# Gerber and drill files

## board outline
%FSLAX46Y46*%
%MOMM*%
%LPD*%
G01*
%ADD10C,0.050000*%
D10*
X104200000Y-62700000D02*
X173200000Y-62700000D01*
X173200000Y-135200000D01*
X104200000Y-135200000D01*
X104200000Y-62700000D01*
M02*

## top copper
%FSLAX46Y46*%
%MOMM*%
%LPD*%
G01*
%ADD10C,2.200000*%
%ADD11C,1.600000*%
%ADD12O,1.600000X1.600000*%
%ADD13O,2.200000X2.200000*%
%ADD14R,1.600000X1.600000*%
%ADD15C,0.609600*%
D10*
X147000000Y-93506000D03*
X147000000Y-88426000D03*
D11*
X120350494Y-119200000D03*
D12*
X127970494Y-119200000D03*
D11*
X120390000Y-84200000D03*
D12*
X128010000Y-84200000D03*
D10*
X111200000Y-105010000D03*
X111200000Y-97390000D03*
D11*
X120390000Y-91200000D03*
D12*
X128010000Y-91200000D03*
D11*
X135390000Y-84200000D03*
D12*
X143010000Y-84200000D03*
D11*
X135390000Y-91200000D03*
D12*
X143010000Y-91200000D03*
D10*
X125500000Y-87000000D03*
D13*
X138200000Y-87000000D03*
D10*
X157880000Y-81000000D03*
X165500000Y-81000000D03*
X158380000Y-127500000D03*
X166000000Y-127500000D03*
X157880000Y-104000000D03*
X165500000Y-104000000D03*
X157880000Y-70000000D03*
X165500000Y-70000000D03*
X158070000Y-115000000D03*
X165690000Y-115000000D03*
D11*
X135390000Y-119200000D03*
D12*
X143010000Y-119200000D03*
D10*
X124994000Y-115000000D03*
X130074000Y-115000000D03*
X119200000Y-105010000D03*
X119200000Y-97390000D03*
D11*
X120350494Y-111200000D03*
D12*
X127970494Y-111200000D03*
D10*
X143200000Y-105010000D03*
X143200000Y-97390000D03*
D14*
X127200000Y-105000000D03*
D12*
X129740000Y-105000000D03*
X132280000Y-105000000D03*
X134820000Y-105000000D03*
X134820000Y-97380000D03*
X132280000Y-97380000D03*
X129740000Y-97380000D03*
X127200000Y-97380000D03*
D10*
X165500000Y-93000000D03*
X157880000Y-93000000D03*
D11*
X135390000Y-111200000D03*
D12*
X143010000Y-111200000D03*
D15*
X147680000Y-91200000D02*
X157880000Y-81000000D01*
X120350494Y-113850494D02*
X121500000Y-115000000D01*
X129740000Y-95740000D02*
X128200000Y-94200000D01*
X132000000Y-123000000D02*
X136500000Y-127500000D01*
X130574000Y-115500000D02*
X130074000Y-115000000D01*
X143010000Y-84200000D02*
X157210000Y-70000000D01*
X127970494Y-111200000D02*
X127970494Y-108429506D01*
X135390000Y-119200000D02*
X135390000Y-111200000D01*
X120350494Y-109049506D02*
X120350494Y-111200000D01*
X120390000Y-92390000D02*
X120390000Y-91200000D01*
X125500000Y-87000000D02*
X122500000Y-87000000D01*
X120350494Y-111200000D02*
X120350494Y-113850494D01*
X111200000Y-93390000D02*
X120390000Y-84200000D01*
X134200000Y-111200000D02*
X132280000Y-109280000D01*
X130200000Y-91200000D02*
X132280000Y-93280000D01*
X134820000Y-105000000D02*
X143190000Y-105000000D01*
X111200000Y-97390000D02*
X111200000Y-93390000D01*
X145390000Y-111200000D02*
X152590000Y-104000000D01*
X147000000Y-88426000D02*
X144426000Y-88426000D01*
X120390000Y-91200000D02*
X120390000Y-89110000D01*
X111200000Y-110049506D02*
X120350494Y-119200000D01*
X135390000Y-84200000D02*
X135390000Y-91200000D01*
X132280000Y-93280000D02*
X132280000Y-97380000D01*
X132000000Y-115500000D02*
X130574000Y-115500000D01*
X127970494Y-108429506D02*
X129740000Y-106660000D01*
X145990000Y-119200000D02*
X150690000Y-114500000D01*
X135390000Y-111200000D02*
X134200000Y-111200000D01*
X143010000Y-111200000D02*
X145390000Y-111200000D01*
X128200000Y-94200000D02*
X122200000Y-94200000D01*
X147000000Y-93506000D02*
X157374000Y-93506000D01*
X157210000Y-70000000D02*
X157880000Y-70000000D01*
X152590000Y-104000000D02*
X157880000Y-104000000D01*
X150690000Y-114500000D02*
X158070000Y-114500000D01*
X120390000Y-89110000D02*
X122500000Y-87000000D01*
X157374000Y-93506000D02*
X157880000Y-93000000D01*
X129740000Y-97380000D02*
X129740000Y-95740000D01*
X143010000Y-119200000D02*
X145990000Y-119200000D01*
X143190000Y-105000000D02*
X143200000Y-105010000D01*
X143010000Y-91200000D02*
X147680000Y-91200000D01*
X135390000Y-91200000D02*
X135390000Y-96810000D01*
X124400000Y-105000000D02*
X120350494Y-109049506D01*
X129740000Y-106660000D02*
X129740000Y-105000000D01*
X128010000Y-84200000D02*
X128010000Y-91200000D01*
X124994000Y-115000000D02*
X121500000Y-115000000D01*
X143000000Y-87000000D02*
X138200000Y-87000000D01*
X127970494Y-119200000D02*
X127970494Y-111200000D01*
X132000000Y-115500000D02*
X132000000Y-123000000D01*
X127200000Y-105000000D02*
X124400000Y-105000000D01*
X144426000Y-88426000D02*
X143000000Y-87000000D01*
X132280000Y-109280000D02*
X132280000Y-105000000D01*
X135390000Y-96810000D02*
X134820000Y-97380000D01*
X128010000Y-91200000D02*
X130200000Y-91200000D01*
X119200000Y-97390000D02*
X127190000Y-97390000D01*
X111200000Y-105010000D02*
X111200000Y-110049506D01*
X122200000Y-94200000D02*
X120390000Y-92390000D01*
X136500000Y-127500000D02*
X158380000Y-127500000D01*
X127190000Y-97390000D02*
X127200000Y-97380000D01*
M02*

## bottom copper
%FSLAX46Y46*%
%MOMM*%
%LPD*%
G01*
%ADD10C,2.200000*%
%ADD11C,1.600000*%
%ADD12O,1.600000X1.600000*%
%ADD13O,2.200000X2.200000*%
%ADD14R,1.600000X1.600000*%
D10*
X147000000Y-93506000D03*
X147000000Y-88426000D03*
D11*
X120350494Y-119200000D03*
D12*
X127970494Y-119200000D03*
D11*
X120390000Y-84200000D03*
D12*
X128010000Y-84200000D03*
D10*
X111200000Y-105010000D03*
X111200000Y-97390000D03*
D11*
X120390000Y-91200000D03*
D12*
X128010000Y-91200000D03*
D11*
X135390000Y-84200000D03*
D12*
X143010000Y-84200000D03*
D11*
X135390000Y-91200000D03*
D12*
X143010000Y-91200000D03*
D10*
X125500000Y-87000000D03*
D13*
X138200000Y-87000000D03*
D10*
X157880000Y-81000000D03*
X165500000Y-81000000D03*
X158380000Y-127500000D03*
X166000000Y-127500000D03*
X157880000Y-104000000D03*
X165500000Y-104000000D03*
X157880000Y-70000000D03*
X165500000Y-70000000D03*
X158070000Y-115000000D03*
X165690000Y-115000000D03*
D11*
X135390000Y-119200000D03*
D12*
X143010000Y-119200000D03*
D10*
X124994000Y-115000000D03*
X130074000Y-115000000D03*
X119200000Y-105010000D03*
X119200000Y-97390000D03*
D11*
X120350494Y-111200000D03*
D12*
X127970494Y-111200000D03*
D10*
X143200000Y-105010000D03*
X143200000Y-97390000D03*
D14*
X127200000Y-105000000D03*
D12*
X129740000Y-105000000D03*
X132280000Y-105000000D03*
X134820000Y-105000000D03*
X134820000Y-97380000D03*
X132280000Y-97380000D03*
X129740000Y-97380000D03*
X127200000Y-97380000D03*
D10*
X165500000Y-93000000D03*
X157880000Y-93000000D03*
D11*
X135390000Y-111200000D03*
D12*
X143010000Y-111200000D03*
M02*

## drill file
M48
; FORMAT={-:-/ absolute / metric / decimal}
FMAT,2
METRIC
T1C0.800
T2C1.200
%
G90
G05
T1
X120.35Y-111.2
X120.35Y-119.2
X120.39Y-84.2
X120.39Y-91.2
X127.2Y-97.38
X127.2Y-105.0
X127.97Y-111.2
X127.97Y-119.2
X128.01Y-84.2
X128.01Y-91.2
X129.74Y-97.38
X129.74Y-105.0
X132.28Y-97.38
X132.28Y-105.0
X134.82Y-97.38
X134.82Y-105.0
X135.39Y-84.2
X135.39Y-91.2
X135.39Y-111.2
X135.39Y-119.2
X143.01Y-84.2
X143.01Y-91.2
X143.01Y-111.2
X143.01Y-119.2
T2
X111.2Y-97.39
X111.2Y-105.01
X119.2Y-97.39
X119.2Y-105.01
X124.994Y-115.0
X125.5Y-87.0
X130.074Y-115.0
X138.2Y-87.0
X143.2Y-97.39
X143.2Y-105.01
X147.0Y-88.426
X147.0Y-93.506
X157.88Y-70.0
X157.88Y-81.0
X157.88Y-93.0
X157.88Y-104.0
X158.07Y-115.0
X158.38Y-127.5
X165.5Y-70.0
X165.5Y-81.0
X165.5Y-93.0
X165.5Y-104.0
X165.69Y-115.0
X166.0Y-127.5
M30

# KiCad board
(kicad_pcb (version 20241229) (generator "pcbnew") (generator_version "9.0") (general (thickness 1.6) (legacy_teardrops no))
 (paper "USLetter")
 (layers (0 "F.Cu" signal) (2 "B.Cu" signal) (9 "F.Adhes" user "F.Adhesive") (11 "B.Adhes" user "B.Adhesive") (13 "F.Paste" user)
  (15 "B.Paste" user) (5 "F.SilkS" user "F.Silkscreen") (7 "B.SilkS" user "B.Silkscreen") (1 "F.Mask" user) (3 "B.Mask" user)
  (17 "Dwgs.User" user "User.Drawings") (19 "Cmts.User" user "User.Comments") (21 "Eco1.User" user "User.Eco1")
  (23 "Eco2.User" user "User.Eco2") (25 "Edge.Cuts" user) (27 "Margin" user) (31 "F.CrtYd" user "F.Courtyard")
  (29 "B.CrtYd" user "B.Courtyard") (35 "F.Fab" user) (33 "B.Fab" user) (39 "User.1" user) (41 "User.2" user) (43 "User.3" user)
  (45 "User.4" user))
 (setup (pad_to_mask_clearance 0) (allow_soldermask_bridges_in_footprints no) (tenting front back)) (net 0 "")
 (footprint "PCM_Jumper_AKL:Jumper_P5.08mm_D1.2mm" (layer "F.Cu") (at 147 93.506 90)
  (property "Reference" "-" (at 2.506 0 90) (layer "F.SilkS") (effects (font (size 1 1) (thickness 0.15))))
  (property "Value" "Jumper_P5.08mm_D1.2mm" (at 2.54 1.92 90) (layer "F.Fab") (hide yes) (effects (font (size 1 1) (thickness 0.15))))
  (pad "1" thru_hole circle (at 0 0 90) (size 2.2 2.2) (drill 1.2) (layers "*.Cu" "*.Mask") (remove_unused_layers no))
  (pad "2" thru_hole circle (at 5.08 0 90) (size 2.2 2.2) (drill 1.2) (layers "*.Cu" "*.Mask") (remove_unused_layers no)))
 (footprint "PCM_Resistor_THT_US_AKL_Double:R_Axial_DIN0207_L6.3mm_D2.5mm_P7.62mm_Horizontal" (layer "F.Cu") (at 120.350494 119.2)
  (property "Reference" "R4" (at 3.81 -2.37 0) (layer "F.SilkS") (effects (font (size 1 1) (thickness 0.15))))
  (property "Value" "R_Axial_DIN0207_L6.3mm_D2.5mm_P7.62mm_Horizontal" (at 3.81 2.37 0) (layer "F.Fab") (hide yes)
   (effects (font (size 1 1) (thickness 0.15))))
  (pad "1" thru_hole circle (at 0 0) (size 1.6 1.6) (drill 0.8) (layers "*.Cu" "*.Mask") (remove_unused_layers no))
  (pad "2" thru_hole oval (at 7.62 0) (size 1.6 1.6) (drill 0.8) (layers "*.Cu" "*.Mask") (remove_unused_layers no)))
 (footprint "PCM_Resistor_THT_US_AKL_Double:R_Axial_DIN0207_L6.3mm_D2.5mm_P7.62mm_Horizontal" (layer "F.Cu") (at 120.39 84.2)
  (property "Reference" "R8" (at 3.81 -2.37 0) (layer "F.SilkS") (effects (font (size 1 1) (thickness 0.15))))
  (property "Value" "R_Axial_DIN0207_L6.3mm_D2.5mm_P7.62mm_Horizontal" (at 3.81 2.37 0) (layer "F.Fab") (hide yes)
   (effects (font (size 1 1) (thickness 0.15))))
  (pad "1" thru_hole circle (at 0 0) (size 1.6 1.6) (drill 0.8) (layers "*.Cu" "*.Mask") (remove_unused_layers no))
  (pad "2" thru_hole oval (at 7.62 0) (size 1.6 1.6) (drill 0.8) (layers "*.Cu" "*.Mask") (remove_unused_layers no)))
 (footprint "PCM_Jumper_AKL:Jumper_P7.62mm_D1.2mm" (layer "F.Cu") (at 111.2 105.01 90)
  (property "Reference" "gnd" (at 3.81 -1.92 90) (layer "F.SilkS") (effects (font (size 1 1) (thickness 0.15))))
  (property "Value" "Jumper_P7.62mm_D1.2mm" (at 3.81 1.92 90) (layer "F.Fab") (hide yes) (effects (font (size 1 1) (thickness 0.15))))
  (pad "1" thru_hole circle (at 0 0 90) (size 2.2 2.2) (drill 1.2) (layers "*.Cu" "*.Mask") (remove_unused_layers no))
  (pad "2" thru_hole circle (at 7.62 0 90) (size 2.2 2.2) (drill 1.2) (layers "*.Cu" "*.Mask") (remove_unused_layers no)))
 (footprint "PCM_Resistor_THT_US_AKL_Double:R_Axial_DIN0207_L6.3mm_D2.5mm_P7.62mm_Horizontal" (layer "F.Cu") (at 120.39 91.2)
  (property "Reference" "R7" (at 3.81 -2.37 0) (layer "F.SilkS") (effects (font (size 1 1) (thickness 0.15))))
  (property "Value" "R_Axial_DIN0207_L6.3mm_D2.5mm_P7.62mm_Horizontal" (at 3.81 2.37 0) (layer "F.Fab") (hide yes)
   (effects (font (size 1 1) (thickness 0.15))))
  (pad "1" thru_hole circle (at 0 0) (size 1.6 1.6) (drill 0.8) (layers "*.Cu" "*.Mask") (remove_unused_layers no))
  (pad "2" thru_hole oval (at 7.62 0) (size 1.6 1.6) (drill 0.8) (layers "*.Cu" "*.Mask") (remove_unused_layers no)))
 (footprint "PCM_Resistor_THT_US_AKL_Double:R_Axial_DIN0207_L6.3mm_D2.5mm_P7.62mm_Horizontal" (layer "F.Cu") (at 135.39 84.2)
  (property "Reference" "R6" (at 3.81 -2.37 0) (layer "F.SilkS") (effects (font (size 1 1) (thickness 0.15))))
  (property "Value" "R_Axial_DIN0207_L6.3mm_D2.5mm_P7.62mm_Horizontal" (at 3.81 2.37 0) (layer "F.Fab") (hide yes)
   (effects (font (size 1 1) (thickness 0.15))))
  (pad "1" thru_hole circle (at 0 0) (size 1.6 1.6) (drill 0.8) (layers "*.Cu" "*.Mask") (remove_unused_layers no))
  (pad "2" thru_hole oval (at 7.62 0) (size 1.6 1.6) (drill 0.8) (layers "*.Cu" "*.Mask") (remove_unused_layers no)))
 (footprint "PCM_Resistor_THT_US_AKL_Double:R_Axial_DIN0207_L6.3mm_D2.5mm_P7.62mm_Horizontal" (layer "F.Cu") (at 135.39 91.2)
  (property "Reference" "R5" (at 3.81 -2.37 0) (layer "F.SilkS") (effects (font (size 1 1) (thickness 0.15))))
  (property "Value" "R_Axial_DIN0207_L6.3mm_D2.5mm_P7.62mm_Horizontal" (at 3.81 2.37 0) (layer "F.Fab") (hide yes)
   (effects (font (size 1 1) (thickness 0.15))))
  (pad "1" thru_hole circle (at 0 0) (size 1.6 1.6) (drill 0.8) (layers "*.Cu" "*.Mask") (remove_unused_layers no))
  (pad "2" thru_hole oval (at 7.62 0) (size 1.6 1.6) (drill 0.8) (layers "*.Cu" "*.Mask") (remove_unused_layers no)))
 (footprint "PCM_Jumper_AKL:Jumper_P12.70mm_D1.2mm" (layer "F.Cu") (at 125.5 87)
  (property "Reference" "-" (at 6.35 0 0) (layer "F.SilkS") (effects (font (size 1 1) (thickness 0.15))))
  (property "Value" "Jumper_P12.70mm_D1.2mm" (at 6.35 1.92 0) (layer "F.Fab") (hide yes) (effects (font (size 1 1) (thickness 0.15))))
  (pad "1" thru_hole circle (at 0 0) (size 2.2 2.2) (drill 1.2) (layers "*.Cu" "*.Mask") (remove_unused_layers no))
  (pad "2" thru_hole oval (at 12.7 0) (size 2.2 2.2) (drill 1.2) (layers "*.Cu" "*.Mask") (remove_unused_layers no)))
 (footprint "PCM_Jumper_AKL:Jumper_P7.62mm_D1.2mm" (layer "F.Cu") (at 157.88 81)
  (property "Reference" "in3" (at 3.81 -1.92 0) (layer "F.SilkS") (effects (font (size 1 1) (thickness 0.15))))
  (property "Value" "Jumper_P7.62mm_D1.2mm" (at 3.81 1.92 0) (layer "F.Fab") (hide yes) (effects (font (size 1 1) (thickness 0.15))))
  (pad "1" thru_hole circle (at 0 0) (size 2.2 2.2) (drill 1.2) (layers "*.Cu" "*.Mask") (remove_unused_layers no))
  (pad "2" thru_hole circle (at 7.62 0) (size 2.2 2.2) (drill 1.2) (layers "*.Cu" "*.Mask") (remove_unused_layers no)))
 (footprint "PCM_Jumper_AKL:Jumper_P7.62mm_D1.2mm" (layer "F.Cu") (at 158.38 127.5)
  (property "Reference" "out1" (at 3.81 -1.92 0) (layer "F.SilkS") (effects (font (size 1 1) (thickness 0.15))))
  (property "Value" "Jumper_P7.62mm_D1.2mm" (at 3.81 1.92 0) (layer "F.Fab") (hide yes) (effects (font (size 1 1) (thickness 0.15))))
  (pad "1" thru_hole circle (at 0 0) (size 2.2 2.2) (drill 1.2) (layers "*.Cu" "*.Mask") (remove_unused_layers no))
  (pad "2" thru_hole circle (at 7.62 0) (size 2.2 2.2) (drill 1.2) (layers "*.Cu" "*.Mask") (remove_unused_layers no)))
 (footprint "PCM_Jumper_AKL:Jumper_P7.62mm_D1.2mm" (layer "F.Cu") (at 157.88 104)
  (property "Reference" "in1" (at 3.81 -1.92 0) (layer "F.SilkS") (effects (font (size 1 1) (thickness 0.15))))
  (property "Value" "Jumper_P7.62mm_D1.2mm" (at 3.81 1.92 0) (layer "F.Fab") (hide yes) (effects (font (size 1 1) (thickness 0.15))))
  (pad "1" thru_hole circle (at 0 0) (size 2.2 2.2) (drill 1.2) (layers "*.Cu" "*.Mask") (remove_unused_layers no))
  (pad "2" thru_hole circle (at 7.62 0) (size 2.2 2.2) (drill 1.2) (layers "*.Cu" "*.Mask") (remove_unused_layers no)))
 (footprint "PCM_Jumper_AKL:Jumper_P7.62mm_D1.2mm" (layer "F.Cu") (at 157.88 70)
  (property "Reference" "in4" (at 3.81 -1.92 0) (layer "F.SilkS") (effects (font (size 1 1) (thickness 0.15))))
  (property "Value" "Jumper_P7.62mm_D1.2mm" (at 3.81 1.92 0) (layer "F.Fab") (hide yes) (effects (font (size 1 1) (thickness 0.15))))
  (pad "1" thru_hole circle (at 0 0) (size 2.2 2.2) (drill 1.2) (layers "*.Cu" "*.Mask") (remove_unused_layers no))
  (pad "2" thru_hole circle (at 7.62 0) (size 2.2 2.2) (drill 1.2) (layers "*.Cu" "*.Mask") (remove_unused_layers no)))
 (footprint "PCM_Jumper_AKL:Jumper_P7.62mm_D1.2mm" (layer "F.Cu") (at 158.07 115)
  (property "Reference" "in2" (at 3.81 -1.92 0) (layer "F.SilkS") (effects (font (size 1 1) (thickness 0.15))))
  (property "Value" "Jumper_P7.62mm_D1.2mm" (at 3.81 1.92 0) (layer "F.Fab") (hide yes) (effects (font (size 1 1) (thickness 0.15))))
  (pad "1" thru_hole circle (at 0 0) (size 2.2 2.2) (drill 1.2) (layers "*.Cu" "*.Mask") (remove_unused_layers no))
  (pad "2" thru_hole circle (at 7.62 0) (size 2.2 2.2) (drill 1.2) (layers "*.Cu" "*.Mask") (remove_unused_layers no)))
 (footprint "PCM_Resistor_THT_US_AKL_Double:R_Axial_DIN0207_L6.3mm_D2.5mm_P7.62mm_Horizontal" (layer "F.Cu") (at 135.39 119.2)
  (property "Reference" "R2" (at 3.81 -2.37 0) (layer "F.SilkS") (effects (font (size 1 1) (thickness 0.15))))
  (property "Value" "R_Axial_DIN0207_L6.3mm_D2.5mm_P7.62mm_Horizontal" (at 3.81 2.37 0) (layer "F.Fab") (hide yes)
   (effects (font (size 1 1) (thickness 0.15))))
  (pad "1" thru_hole circle (at 0 0) (size 1.6 1.6) (drill 0.8) (layers "*.Cu" "*.Mask") (remove_unused_layers no))
  (pad "2" thru_hole oval (at 7.62 0) (size 1.6 1.6) (drill 0.8) (layers "*.Cu" "*.Mask") (remove_unused_layers no)))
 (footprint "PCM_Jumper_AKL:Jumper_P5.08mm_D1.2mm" (layer "F.Cu") (at 124.994 115)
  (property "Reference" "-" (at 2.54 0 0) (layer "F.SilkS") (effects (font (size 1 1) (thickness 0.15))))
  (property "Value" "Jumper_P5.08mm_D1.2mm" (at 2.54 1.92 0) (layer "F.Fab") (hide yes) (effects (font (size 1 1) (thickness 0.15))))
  (pad "1" thru_hole circle (at 0 0) (size 2.2 2.2) (drill 1.2) (layers "*.Cu" "*.Mask") (remove_unused_layers no))
  (pad "2" thru_hole circle (at 5.08 0) (size 2.2 2.2) (drill 1.2) (layers "*.Cu" "*.Mask") (remove_unused_layers no)))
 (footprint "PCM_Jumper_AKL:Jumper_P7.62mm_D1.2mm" (layer "F.Cu") (at 119.2 105.01 90)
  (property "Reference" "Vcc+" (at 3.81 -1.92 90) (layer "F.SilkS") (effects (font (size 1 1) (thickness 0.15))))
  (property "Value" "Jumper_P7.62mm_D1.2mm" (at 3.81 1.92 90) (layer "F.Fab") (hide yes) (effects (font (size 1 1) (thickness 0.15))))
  (pad "1" thru_hole circle (at 0 0 90) (size 2.2 2.2) (drill 1.2) (layers "*.Cu" "*.Mask") (remove_unused_layers no))
  (pad "2" thru_hole circle (at 7.62 0 90) (size 2.2 2.2) (drill 1.2) (layers "*.Cu" "*.Mask") (remove_unused_layers no)))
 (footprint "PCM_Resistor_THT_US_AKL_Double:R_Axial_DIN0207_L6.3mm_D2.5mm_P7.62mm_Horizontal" (layer "F.Cu") (at 120.350494 111.2)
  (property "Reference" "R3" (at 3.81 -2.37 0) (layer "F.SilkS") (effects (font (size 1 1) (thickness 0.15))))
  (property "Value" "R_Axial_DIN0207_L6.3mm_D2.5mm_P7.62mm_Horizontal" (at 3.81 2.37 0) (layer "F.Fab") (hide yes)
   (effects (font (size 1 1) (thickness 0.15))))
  (pad "1" thru_hole circle (at 0 0) (size 1.6 1.6) (drill 0.8) (layers "*.Cu" "*.Mask") (remove_unused_layers no))
  (pad "2" thru_hole oval (at 7.62 0) (size 1.6 1.6) (drill 0.8) (layers "*.Cu" "*.Mask") (remove_unused_layers no)))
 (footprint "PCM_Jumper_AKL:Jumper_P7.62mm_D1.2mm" (layer "F.Cu") (at 143.2 105.01 90)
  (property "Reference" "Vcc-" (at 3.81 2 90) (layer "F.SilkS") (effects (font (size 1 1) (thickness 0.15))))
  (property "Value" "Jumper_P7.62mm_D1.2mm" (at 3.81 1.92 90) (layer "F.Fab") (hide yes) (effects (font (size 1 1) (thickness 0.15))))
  (pad "1" thru_hole circle (at 0 0 90) (size 2.2 2.2) (drill 1.2) (layers "*.Cu" "*.Mask") (remove_unused_layers no))
  (pad "2" thru_hole circle (at 7.62 0 90) (size 2.2 2.2) (drill 1.2) (layers "*.Cu" "*.Mask") (remove_unused_layers no)))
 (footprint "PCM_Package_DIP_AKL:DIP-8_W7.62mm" (layer "F.Cu") (at 127.2 105 90)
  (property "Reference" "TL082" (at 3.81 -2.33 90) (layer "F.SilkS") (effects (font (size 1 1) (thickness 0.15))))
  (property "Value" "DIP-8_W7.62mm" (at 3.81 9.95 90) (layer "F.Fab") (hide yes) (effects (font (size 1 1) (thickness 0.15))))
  (pad "1" thru_hole rect (at 0 0 90) (size 1.6 1.6) (drill 0.8) (layers "*.Cu" "*.Mask") (remove_unused_layers no))
  (pad "2" thru_hole oval (at 0 2.54 90) (size 1.6 1.6) (drill 0.8) (layers "*.Cu" "*.Mask") (remove_unused_layers no))
  (pad "3" thru_hole oval (at 0 5.08 90) (size 1.6 1.6) (drill 0.8) (layers "*.Cu" "*.Mask") (remove_unused_layers no))
  (pad "4" thru_hole oval (at 0 7.62 90) (size 1.6 1.6) (drill 0.8) (layers "*.Cu" "*.Mask") (remove_unused_layers no))
  (pad "5" thru_hole oval (at 7.62 7.62 90) (size 1.6 1.6) (drill 0.8) (layers "*.Cu" "*.Mask") (remove_unused_layers no))
  (pad "6" thru_hole oval (at 7.62 5.08 90) (size 1.6 1.6) (drill 0.8) (layers "*.Cu" "*.Mask") (remove_unused_layers no))
  (pad "7" thru_hole oval (at 7.62 2.54 90) (size 1.6 1.6) (drill 0.8) (layers "*.Cu" "*.Mask") (remove_unused_layers no))
  (pad "8" thru_hole oval (at 7.62 0 90) (size 1.6 1.6) (drill 0.8) (layers "*.Cu" "*.Mask") (remove_unused_layers no)))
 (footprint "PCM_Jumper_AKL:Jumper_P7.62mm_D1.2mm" (layer "F.Cu") (at 165.5 93 180)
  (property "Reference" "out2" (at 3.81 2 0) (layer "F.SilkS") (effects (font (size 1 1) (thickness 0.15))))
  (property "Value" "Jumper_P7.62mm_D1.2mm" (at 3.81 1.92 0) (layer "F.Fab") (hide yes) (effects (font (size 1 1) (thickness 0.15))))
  (pad "1" thru_hole circle (at 0 0 180) (size 2.2 2.2) (drill 1.2) (layers "*.Cu" "*.Mask") (remove_unused_layers no))
  (pad "2" thru_hole circle (at 7.62 0 180) (size 2.2 2.2) (drill 1.2) (layers "*.Cu" "*.Mask") (remove_unused_layers no)))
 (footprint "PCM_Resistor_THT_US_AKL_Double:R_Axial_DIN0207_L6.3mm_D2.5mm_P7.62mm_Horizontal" (layer "F.Cu") (at 135.39 111.2)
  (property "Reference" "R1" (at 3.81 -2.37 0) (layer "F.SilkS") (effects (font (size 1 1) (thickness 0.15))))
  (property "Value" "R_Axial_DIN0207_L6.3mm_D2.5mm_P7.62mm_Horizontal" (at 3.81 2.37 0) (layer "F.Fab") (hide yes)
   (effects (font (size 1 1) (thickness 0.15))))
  (pad "1" thru_hole circle (at 0 0) (size 1.6 1.6) (drill 0.8) (layers "*.Cu" "*.Mask") (remove_unused_layers no))
  (pad "2" thru_hole oval (at 7.62 0) (size 1.6 1.6) (drill 0.8) (layers "*.Cu" "*.Mask") (remove_unused_layers no)))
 (gr_rect (start 104.2 62.7) (end 173.2 135.2) (stroke (width 0.05) (type default)) (fill no) (layer "Edge.Cuts"))
 (segment (start 147.68 91.2) (end 157.88 81) (width 0.6096) (layer "F.Cu") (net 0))
 (segment (start 120.350494 113.850494) (end 121.5 115) (width 0.6096) (layer "F.Cu") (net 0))
 (segment (start 129.74 95.74) (end 128.2 94.2) (width 0.6096) (layer "F.Cu") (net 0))
 (segment (start 132 123) (end 136.5 127.5) (width 0.6096) (layer "F.Cu") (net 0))
 (segment (start 130.574 115.5) (end 130.074 115) (width 0.6096) (layer "F.Cu") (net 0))
 (segment (start 143.01 84.2) (end 157.21 70) (width 0.6096) (layer "F.Cu") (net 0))
 (segment (start 127.970494 111.2) (end 127.970494 108.429506) (width 0.6096) (layer "F.Cu") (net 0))
 (segment (start 135.39 119.2) (end 135.39 111.2) (width 0.6096) (layer "F.Cu") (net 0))
 (segment (start 120.350494 109.049506) (end 120.350494 111.2) (width 0.6096) (layer "F.Cu") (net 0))
 (segment (start 120.39 92.39) (end 120.39 91.2) (width 0.6096) (layer "F.Cu") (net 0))
 (segment (start 125.5 87) (end 122.5 87) (width 0.6096) (layer "F.Cu") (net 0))
 (segment (start 120.350494 111.2) (end 120.350494 113.850494) (width 0.6096) (layer "F.Cu") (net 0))
 (segment (start 111.2 93.39) (end 120.39 84.2) (width 0.6096) (layer "F.Cu") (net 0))
 (segment (start 134.2 111.2) (end 132.28 109.28) (width 0.6096) (layer "F.Cu") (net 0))
 (segment (start 130.2 91.2) (end 132.28 93.28) (width 0.6096) (layer "F.Cu") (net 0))
 (segment (start 134.82 105) (end 143.19 105) (width 0.6096) (layer "F.Cu") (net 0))
 (segment (start 111.2 97.39) (end 111.2 93.39) (width 0.6096) (layer "F.Cu") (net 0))
 (segment (start 145.39 111.2) (end 152.59 104) (width 0.6096) (layer "F.Cu") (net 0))
 (segment (start 147 88.426) (end 144.426 88.426) (width 0.6096) (layer "F.Cu") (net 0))
 (segment (start 120.39 91.2) (end 120.39 89.11) (width 0.6096) (layer "F.Cu") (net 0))
 (segment (start 111.2 110.049506) (end 120.350494 119.2) (width 0.6096) (layer "F.Cu") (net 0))
 (segment (start 135.39 84.2) (end 135.39 91.2) (width 0.6096) (layer "F.Cu") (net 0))
 (segment (start 132.28 93.28) (end 132.28 97.38) (width 0.6096) (layer "F.Cu") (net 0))
 (segment (start 132 115.5) (end 130.574 115.5) (width 0.6096) (layer "F.Cu") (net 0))
 (segment (start 127.970494 108.429506) (end 129.74 106.66) (width 0.6096) (layer "F.Cu") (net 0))
 (segment (start 145.99 119.2) (end 150.69 114.5) (width 0.6096) (layer "F.Cu") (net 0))
 (segment (start 135.39 111.2) (end 134.2 111.2) (width 0.6096) (layer "F.Cu") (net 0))
 (segment (start 143.01 111.2) (end 145.39 111.2) (width 0.6096) (layer "F.Cu") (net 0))
 (segment (start 128.2 94.2) (end 122.2 94.2) (width 0.6096) (layer "F.Cu") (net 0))
 (segment (start 147 93.506) (end 157.374 93.506) (width 0.6096) (layer "F.Cu") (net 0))
 (segment (start 157.21 70) (end 157.88 70) (width 0.6096) (layer "F.Cu") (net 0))
 (segment (start 152.59 104) (end 157.88 104) (width 0.6096) (layer "F.Cu") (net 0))
 (segment (start 150.69 114.5) (end 158.07 114.5) (width 0.6096) (layer "F.Cu") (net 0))
 (segment (start 120.39 89.11) (end 122.5 87) (width 0.6096) (layer "F.Cu") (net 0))
 (segment (start 157.374 93.506) (end 157.88 93) (width 0.6096) (layer "F.Cu") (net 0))
 (segment (start 129.74 97.38) (end 129.74 95.74) (width 0.6096) (layer "F.Cu") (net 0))
 (segment (start 143.01 119.2) (end 145.99 119.2) (width 0.6096) (layer "F.Cu") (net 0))
 (segment (start 143.19 105) (end 143.2 105.01) (width 0.6096) (layer "F.Cu") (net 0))
 (segment (start 143.01 91.2) (end 147.68 91.2) (width 0.6096) (layer "F.Cu") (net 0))
 (segment (start 135.39 91.2) (end 135.39 96.81) (width 0.6096) (layer "F.Cu") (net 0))
 (segment (start 124.4 105) (end 120.350494 109.049506) (width 0.6096) (layer "F.Cu") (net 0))
 (segment (start 129.74 106.66) (end 129.74 105) (width 0.6096) (layer "F.Cu") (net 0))
 (segment (start 128.01 84.2) (end 128.01 91.2) (width 0.6096) (layer "F.Cu") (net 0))
 (segment (start 124.994 115) (end 121.5 115) (width 0.6096) (layer "F.Cu") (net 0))
 (segment (start 143 87) (end 138.2 87) (width 0.6096) (layer "F.Cu") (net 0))
 (segment (start 127.970494 119.2) (end 127.970494 111.2) (width 0.6096) (layer "F.Cu") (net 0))
 (segment (start 132 115.5) (end 132 123) (width 0.6096) (layer "F.Cu") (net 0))
 (segment (start 127.2 105) (end 124.4 105) (width 0.6096) (layer "F.Cu") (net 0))
 (segment (start 144.426 88.426) (end 143 87) (width 0.6096) (layer "F.Cu") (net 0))
 (segment (start 132.28 109.28) (end 132.28 105) (width 0.6096) (layer "F.Cu") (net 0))
 (segment (start 135.39 96.81) (end 134.82 97.38) (width 0.6096) (layer "F.Cu") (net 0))
 (segment (start 128.01 91.2) (end 130.2 91.2) (width 0.6096) (layer "F.Cu") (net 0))
 (segment (start 119.2 97.39) (end 127.19 97.39) (width 0.6096) (layer "F.Cu") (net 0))
 (segment (start 111.2 105.01) (end 111.2 110.049506) (width 0.6096) (layer "F.Cu") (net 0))
 (segment (start 122.2 94.2) (end 120.39 92.39) (width 0.6096) (layer "F.Cu") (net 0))
 (segment (start 136.5 127.5) (end 158.38 127.5) (width 0.6096) (layer "F.Cu") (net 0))
 (segment (start 127.19 97.39) (end 127.2 97.38) (width 0.6096) (layer "F.Cu") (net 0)))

